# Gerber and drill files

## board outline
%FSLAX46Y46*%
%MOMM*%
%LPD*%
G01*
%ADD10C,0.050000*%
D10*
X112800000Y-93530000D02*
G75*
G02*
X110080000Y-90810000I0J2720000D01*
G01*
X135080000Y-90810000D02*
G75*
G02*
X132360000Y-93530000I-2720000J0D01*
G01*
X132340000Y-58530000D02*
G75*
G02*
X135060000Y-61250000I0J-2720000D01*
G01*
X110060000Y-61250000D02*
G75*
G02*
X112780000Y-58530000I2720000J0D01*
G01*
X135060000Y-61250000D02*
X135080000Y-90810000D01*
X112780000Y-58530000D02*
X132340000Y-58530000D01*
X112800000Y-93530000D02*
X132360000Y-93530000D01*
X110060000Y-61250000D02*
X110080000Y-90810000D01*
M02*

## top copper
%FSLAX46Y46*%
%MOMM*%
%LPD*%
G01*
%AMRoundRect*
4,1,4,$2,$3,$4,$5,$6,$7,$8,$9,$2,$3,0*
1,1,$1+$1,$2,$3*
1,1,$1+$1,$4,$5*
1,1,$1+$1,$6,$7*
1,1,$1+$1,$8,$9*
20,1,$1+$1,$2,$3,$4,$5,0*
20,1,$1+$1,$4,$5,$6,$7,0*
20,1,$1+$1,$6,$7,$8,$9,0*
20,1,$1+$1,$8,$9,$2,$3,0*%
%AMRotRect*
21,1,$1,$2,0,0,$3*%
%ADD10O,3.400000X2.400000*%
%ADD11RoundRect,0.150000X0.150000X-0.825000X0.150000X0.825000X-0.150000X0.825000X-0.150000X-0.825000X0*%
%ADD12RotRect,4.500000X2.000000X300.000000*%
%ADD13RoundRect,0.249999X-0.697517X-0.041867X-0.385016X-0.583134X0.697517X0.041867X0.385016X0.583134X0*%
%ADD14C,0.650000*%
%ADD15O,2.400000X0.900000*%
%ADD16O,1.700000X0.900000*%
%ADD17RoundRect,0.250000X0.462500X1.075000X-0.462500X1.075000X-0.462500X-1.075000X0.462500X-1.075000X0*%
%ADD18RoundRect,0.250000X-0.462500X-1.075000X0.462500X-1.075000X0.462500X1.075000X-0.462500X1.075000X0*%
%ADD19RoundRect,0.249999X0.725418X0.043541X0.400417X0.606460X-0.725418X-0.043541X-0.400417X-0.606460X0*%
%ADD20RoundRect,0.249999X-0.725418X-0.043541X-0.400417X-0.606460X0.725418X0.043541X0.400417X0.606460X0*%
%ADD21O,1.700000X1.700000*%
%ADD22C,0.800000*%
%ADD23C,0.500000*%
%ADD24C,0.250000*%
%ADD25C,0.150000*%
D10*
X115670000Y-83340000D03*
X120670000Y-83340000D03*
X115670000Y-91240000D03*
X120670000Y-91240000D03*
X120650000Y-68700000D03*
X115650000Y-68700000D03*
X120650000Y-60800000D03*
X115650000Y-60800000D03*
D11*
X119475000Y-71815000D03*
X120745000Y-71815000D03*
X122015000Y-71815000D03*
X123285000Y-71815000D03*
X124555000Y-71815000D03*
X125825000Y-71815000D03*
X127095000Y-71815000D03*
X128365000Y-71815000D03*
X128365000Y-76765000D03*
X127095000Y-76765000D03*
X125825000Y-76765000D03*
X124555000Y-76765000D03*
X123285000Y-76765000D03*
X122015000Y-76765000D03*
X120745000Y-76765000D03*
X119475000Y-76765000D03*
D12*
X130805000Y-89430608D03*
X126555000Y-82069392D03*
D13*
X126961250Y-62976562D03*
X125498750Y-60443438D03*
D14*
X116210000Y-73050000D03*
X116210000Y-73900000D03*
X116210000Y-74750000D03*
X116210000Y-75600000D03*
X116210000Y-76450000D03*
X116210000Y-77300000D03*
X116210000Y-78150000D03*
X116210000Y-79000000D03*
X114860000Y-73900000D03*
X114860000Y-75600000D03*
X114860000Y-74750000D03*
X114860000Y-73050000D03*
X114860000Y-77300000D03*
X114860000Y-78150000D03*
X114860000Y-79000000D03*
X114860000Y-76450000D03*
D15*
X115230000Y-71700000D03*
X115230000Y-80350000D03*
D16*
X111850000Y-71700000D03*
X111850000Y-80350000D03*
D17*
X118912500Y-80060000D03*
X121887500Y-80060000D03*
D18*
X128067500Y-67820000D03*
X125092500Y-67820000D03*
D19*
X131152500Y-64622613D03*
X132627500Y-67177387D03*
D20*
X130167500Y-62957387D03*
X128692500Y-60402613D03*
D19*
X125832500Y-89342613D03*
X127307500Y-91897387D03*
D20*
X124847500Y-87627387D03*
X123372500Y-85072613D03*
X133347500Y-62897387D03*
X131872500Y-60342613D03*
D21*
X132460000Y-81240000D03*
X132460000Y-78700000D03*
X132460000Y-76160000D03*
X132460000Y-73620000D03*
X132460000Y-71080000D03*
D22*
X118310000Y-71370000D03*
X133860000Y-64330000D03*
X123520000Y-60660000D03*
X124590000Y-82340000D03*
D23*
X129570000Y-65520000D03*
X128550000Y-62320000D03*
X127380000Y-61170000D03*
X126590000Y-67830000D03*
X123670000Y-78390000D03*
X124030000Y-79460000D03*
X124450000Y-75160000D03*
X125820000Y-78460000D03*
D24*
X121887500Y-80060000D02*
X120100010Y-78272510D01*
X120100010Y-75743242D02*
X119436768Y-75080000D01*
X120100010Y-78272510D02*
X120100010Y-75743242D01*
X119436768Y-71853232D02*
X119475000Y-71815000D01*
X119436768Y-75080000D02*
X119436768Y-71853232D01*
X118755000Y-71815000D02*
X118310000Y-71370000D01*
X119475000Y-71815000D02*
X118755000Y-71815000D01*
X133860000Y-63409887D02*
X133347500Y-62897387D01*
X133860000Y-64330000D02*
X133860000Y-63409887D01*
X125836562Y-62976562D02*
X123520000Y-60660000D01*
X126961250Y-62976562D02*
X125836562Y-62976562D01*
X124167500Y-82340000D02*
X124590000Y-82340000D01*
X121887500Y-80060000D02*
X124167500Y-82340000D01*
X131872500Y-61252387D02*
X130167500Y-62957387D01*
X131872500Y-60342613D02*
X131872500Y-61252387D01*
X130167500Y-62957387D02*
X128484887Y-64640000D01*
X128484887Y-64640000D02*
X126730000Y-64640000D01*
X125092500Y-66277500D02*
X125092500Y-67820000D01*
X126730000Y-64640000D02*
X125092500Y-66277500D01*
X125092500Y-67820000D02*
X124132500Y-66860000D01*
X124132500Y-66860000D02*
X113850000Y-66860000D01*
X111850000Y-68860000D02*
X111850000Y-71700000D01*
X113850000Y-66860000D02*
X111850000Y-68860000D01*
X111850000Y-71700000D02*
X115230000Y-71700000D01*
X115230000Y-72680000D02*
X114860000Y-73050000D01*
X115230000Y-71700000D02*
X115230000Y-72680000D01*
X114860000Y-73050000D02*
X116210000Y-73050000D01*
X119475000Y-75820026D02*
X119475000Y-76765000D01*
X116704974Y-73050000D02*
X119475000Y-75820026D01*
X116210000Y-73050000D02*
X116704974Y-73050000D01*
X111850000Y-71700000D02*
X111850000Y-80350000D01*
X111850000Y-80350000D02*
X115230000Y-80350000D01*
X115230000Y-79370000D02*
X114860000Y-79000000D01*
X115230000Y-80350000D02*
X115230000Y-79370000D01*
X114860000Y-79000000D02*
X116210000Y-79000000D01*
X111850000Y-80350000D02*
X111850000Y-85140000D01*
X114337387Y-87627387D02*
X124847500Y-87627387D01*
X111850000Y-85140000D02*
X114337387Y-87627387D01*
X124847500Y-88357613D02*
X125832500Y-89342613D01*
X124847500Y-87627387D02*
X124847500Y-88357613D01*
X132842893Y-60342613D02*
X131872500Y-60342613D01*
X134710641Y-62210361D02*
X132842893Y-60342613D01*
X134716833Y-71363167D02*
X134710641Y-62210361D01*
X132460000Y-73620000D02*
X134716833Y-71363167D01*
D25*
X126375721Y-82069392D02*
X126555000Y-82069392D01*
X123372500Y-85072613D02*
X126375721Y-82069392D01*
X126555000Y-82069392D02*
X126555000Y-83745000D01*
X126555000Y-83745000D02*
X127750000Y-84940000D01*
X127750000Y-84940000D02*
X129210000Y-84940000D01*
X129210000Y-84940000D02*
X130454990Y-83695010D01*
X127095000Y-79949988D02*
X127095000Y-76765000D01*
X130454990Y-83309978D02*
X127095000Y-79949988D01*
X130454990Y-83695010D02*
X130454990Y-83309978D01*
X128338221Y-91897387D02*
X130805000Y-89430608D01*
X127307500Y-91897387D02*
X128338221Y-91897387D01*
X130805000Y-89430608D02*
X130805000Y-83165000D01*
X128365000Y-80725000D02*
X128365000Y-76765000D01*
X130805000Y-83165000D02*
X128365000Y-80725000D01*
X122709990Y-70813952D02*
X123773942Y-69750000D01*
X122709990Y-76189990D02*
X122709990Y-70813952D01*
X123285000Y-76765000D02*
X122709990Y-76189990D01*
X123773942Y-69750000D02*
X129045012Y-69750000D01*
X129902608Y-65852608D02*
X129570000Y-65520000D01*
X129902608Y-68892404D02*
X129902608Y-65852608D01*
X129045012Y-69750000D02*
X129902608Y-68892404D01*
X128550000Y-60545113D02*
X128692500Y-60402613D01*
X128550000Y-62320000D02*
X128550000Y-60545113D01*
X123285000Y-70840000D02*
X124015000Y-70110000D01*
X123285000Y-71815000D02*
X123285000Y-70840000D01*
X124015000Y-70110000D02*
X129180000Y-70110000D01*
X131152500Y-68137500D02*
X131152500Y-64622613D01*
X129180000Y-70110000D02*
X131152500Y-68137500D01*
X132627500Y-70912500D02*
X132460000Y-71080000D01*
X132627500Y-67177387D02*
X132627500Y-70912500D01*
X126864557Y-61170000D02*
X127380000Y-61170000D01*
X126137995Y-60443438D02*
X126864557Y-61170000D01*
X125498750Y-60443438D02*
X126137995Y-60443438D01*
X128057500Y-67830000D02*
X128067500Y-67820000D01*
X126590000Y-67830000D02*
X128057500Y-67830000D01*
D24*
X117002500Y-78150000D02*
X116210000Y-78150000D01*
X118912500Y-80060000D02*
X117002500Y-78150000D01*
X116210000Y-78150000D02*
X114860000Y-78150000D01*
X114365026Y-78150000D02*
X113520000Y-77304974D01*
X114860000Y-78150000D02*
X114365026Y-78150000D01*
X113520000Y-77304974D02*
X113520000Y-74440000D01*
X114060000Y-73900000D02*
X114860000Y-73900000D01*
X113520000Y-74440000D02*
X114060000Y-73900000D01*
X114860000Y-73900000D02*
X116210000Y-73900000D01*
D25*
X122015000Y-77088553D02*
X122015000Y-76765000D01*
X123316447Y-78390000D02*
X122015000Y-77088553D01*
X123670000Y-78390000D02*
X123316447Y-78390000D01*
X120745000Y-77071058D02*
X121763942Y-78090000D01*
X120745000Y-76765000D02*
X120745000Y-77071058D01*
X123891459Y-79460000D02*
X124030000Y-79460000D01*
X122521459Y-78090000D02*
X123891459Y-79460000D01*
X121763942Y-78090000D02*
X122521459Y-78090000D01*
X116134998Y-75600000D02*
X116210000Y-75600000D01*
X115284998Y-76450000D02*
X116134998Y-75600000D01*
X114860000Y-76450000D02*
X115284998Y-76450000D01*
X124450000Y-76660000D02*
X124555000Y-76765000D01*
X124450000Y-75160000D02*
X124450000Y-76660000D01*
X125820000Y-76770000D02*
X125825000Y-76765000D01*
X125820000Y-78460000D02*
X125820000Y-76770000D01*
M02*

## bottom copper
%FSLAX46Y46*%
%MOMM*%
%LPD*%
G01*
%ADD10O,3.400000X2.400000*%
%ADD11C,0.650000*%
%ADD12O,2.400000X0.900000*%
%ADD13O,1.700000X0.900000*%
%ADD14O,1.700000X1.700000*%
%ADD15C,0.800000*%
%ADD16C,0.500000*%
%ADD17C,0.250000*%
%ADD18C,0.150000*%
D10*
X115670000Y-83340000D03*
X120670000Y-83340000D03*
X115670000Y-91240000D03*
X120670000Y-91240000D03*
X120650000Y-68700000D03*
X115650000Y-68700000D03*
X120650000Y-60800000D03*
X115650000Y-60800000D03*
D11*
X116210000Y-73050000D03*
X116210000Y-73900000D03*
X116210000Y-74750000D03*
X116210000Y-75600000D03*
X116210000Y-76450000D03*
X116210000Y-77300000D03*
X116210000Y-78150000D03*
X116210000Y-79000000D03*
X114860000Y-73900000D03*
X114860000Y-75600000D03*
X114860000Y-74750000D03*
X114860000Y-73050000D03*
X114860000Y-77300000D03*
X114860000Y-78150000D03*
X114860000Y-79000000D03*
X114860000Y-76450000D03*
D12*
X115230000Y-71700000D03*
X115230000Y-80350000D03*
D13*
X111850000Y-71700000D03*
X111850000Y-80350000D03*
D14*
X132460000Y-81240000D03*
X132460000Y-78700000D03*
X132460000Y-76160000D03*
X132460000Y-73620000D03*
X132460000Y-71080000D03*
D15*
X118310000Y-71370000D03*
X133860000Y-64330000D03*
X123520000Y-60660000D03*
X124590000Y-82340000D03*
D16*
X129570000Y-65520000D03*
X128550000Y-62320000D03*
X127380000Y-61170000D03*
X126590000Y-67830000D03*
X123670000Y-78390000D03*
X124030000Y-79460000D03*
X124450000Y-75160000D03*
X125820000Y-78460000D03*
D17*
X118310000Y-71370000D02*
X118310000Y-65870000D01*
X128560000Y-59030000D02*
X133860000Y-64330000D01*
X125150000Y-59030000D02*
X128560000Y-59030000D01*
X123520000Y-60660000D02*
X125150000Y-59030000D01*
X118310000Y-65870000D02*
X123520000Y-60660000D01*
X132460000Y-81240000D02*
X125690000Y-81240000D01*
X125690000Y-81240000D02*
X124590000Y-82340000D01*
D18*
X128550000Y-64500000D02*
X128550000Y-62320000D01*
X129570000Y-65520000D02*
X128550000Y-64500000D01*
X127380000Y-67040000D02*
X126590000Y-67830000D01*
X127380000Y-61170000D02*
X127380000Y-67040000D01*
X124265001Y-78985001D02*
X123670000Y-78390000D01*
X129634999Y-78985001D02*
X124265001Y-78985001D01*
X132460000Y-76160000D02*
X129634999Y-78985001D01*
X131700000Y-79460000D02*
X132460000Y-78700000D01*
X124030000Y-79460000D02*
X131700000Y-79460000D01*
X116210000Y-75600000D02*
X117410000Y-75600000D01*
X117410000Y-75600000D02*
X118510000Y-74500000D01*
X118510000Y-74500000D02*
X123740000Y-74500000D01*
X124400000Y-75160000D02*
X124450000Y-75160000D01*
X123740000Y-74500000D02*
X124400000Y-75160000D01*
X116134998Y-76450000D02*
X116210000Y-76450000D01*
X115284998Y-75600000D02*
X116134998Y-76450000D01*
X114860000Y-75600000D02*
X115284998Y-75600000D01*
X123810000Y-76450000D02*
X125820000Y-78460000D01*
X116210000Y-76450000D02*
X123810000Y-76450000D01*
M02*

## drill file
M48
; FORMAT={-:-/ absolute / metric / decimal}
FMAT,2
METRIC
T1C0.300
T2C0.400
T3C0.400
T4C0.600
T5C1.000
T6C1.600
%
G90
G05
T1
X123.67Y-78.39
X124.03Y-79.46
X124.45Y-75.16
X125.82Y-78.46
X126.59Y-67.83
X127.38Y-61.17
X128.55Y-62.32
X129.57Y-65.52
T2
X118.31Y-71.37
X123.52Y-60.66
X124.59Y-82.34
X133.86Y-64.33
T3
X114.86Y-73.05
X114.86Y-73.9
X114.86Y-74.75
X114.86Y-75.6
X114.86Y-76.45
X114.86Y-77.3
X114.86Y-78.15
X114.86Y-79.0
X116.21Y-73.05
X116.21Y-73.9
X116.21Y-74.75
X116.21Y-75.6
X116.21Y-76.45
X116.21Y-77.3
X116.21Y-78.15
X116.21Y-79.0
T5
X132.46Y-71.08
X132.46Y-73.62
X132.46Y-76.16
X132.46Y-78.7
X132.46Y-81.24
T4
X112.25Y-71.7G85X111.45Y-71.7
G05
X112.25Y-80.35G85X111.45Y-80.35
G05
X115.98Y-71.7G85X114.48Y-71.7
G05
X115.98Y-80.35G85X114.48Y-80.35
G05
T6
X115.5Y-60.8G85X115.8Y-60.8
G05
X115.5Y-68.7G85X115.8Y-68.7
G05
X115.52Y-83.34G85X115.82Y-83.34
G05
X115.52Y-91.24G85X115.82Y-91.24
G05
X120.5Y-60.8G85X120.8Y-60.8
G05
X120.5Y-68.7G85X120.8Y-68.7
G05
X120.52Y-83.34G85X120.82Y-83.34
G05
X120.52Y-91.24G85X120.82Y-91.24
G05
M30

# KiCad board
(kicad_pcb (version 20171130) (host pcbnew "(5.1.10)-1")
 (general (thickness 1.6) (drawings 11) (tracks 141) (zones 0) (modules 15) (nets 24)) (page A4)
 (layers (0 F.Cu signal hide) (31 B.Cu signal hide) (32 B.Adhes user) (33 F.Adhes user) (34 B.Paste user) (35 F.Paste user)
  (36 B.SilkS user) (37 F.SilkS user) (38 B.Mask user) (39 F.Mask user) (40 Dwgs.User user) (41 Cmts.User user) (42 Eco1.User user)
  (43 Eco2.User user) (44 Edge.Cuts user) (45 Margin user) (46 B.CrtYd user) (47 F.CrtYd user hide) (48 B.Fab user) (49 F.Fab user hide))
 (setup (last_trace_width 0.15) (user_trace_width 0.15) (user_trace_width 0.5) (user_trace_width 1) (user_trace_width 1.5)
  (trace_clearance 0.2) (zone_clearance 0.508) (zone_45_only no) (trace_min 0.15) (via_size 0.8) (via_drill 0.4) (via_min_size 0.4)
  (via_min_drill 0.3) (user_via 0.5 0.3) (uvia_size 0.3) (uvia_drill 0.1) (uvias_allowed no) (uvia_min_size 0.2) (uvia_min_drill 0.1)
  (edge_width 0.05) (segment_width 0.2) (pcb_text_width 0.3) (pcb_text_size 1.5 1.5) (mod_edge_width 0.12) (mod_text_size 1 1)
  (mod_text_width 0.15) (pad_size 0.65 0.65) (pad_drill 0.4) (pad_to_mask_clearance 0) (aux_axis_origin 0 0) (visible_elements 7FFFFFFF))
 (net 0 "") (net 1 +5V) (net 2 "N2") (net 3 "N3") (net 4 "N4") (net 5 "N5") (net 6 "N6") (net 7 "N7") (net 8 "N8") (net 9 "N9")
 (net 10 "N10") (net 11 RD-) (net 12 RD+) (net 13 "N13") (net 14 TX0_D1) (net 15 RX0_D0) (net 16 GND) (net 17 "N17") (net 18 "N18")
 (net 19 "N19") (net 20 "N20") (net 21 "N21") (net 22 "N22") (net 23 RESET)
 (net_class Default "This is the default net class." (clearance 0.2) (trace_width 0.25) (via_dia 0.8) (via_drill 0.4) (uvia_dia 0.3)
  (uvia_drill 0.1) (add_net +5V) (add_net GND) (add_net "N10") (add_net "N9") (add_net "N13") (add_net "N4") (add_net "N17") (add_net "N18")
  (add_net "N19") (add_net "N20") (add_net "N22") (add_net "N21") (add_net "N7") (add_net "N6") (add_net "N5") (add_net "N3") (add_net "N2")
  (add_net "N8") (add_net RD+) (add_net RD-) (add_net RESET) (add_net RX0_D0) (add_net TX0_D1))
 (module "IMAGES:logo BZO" (layer B.Cu) (at 123.61 76.22 150)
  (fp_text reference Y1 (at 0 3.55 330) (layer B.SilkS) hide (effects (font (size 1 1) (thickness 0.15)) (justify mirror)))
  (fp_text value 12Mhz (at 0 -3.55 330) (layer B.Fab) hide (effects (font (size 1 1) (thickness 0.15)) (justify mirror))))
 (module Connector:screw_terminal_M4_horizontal (layer F.Cu) (at 115.67 83.54)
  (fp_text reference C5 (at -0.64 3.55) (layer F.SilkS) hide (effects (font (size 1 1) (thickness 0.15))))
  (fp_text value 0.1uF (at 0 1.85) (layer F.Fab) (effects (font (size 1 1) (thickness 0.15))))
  (pad 1 thru_hole oval (at 0 -0.2) (size 3.4 2.4) (drill oval 1.9 1.6) (layers *.Cu *.Mask))
  (pad 2 thru_hole oval (at 5 -0.2) (size 3.4 2.4) (drill oval 1.9 1.6) (layers *.Cu *.Mask))
  (pad 3 thru_hole oval (at 0 7.7) (size 3.4 2.4) (drill oval 1.9 1.6) (layers *.Cu *.Mask))
  (pad 4 thru_hole oval (at 5 7.7) (size 3.4 2.4) (drill oval 1.9 1.6) (layers *.Cu *.Mask)))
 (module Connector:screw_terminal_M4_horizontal (layer F.Cu) (at 115.65 61)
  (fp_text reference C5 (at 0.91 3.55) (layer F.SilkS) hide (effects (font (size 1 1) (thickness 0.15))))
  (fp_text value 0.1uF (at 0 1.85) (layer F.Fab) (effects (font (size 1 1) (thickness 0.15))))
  (pad 4 thru_hole oval (at 5 7.7) (size 3.4 2.4) (drill oval 1.9 1.6) (layers *.Cu *.Mask))
  (pad 3 thru_hole oval (at 0 7.7) (size 3.4 2.4) (drill oval 1.9 1.6) (layers *.Cu *.Mask))
  (pad 2 thru_hole oval (at 5 -0.2) (size 3.4 2.4) (drill oval 1.9 1.6) (layers *.Cu *.Mask))
  (pad 1 thru_hole oval (at 0 -0.2) (size 3.4 2.4) (drill oval 1.9 1.6) (layers *.Cu *.Mask)))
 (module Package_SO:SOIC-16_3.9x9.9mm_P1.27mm (layer F.Cu) (at 123.92 74.29 90)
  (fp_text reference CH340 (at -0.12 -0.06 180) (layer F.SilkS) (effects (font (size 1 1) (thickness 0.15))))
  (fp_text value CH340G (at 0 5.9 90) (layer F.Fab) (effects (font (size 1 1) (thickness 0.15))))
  (pad 16 smd roundrect (at 2.475 -4.445 90) (size 1.95 0.6) (layers F.Cu F.Paste F.Mask) (roundrect_rratio 0.25) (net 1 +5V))
  (pad 15 smd roundrect (at 2.475 -3.175 90) (size 1.95 0.6) (layers F.Cu F.Paste F.Mask) (roundrect_rratio 0.25) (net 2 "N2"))
  (pad 14 smd roundrect (at 2.475 -1.905 90) (size 1.95 0.6) (layers F.Cu F.Paste F.Mask) (roundrect_rratio 0.25) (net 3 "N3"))
  (pad 13 smd roundrect (at 2.475 -0.635 90) (size 1.95 0.6) (layers F.Cu F.Paste F.Mask) (roundrect_rratio 0.25) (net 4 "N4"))
  (pad 12 smd roundrect (at 2.475 0.635 90) (size 1.95 0.6) (layers F.Cu F.Paste F.Mask) (roundrect_rratio 0.25) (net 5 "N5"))
  (pad 11 smd roundrect (at 2.475 1.905 90) (size 1.95 0.6) (layers F.Cu F.Paste F.Mask) (roundrect_rratio 0.25) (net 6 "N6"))
  (pad 10 smd roundrect (at 2.475 3.175 90) (size 1.95 0.6) (layers F.Cu F.Paste F.Mask) (roundrect_rratio 0.25) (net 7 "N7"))
  (pad 9 smd roundrect (at 2.475 4.445 90) (size 1.95 0.6) (layers F.Cu F.Paste F.Mask) (roundrect_rratio 0.25) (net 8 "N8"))
  (pad 8 smd roundrect (at -2.475 4.445 90) (size 1.95 0.6) (layers F.Cu F.Paste F.Mask) (roundrect_rratio 0.25) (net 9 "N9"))
  (pad 7 smd roundrect (at -2.475 3.175 90) (size 1.95 0.6) (layers F.Cu F.Paste F.Mask) (roundrect_rratio 0.25) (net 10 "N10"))
  (pad 6 smd roundrect (at -2.475 1.905 90) (size 1.95 0.6) (layers F.Cu F.Paste F.Mask) (roundrect_rratio 0.25) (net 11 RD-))
  (pad 5 smd roundrect (at -2.475 0.635 90) (size 1.95 0.6) (layers F.Cu F.Paste F.Mask) (roundrect_rratio 0.25) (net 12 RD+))
  (pad 4 smd roundrect (at -2.475 -0.635 90) (size 1.95 0.6) (layers F.Cu F.Paste F.Mask) (roundrect_rratio 0.25) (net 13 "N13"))
  (pad 3 smd roundrect (at -2.475 -1.905 90) (size 1.95 0.6) (layers F.Cu F.Paste F.Mask) (roundrect_rratio 0.25) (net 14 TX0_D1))
  (pad 2 smd roundrect (at -2.475 -3.175 90) (size 1.95 0.6) (layers F.Cu F.Paste F.Mask) (roundrect_rratio 0.25) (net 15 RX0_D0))
  (pad 1 smd roundrect (at -2.475 -4.445 90) (size 1.95 0.6) (layers F.Cu F.Paste F.Mask) (roundrect_rratio 0.25) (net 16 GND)))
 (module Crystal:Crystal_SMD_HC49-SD (layer F.Cu) (at 128.68 85.75 300)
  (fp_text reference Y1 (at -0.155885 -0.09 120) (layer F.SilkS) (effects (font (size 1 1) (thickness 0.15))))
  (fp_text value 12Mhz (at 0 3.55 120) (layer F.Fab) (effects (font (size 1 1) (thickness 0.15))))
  (pad 2 smd rect (at 4.25 0 300) (size 4.5 2) (layers F.Cu F.Paste F.Mask) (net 9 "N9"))
  (pad 1 smd rect (at -4.25 0 300) (size 4.5 2) (layers F.Cu F.Paste F.Mask) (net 10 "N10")))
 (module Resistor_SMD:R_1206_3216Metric (layer F.Cu) (at 126.23 61.71 300)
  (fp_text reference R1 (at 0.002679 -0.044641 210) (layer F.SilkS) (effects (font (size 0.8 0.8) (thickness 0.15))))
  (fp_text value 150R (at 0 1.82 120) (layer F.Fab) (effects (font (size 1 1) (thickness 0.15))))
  (pad 2 smd roundrect (at 1.4625 0 300) (size 1.125 1.75) (layers F.Cu F.Paste F.Mask) (roundrect_rratio 0.2222213333333333) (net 1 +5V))
  (pad 1 smd roundrect (at -1.4625 0 300) (size 1.125 1.75) (layers F.Cu F.Paste F.Mask) (roundrect_rratio 0.2222213333333333)
   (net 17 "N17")))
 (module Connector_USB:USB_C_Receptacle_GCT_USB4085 (layer F.Cu) (at 116.21 73.05 270)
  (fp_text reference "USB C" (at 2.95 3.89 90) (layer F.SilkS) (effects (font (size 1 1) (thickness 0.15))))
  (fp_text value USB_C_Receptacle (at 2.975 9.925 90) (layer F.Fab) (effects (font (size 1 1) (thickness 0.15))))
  (pad A1 thru_hole circle (at 0 0 270) (size 0.65 0.65) (drill 0.4) (layers *.Cu *.Mask) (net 16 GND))
  (pad A4 thru_hole circle (at 0.85 0 270) (size 0.65 0.65) (drill 0.4) (layers *.Cu *.Mask) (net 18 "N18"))
  (pad A5 thru_hole circle (at 1.7 0 270) (size 0.65 0.65) (drill 0.4) (layers *.Cu *.Mask) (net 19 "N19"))
  (pad A6 thru_hole circle (at 2.55 0 270) (size 0.65 0.65) (drill 0.4) (layers *.Cu *.Mask) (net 12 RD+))
  (pad A7 thru_hole circle (at 3.4 0 270) (size 0.65 0.65) (drill 0.4) (layers *.Cu *.Mask) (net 11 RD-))
  (pad A8 thru_hole circle (at 4.25 0 270) (size 0.65 0.65) (drill 0.4) (layers *.Cu *.Mask) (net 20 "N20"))
  (pad A9 thru_hole circle (at 5.1 0 270) (size 0.65 0.65) (drill 0.4) (layers *.Cu *.Mask) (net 18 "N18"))
  (pad A12 thru_hole circle (at 5.95 0 270) (size 0.65 0.65) (drill 0.4) (layers *.Cu *.Mask) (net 16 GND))
  (pad B9 thru_hole circle (at 0.85 1.35 270) (size 0.65 0.65) (drill 0.4) (layers *.Cu *.Mask) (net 18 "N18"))
  (pad B7 thru_hole circle (at 2.55 1.35 270) (size 0.65 0.65) (drill 0.4) (layers *.Cu *.Mask) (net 11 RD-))
  (pad B8 thru_hole circle (at 1.7 1.35 270) (size 0.65 0.65) (drill 0.4) (layers *.Cu *.Mask) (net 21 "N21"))
  (pad B12 thru_hole circle (at 0 1.35 270) (size 0.65 0.65) (drill 0.4) (layers *.Cu *.Mask) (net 16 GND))
  (pad B5 thru_hole circle (at 4.25 1.35 270) (size 0.65 0.65) (drill 0.4) (layers *.Cu *.Mask) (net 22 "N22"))
  (pad B4 thru_hole circle (at 5.1 1.35 270) (size 0.65 0.65) (drill 0.4) (layers *.Cu *.Mask) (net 18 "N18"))
  (pad B1 thru_hole circle (at 5.95 1.35 270) (size 0.65 0.65) (drill 0.4) (layers *.Cu *.Mask) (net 16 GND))
  (pad B6 thru_hole circle (at 3.4 1.35 270) (size 0.65 0.65) (drill 0.4) (layers *.Cu *.Mask) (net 12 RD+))
  (pad S1 thru_hole oval (at -1.35 0.98 270) (size 0.9 2.4) (drill oval 0.6 2.1) (layers *.Cu *.Mask) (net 16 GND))
  (pad S1 thru_hole oval (at 7.3 0.98 270) (size 0.9 2.4) (drill oval 0.6 2.1) (layers *.Cu *.Mask) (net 16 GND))
  (pad S1 thru_hole oval (at -1.35 4.36 270) (size 0.9 1.7) (drill oval 0.6 1.4) (layers *.Cu *.Mask) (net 16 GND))
  (pad S1 thru_hole oval (at 7.3 4.36 270) (size 0.9 1.7) (drill oval 0.6 1.4) (layers *.Cu *.Mask) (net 16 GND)))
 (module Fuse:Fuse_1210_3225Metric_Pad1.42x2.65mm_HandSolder (layer F.Cu) (at 120.4 80.06 180)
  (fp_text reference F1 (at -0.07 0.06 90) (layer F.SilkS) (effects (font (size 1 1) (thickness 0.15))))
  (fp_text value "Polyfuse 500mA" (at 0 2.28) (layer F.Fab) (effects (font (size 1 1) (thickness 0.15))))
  (pad 2 smd roundrect (at 1.4875 0 180) (size 1.425 2.65) (layers F.Cu F.Paste F.Mask) (roundrect_rratio 0.1754385964912281) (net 18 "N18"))
  (pad 1 smd roundrect (at -1.4875 0 180) (size 1.425 2.65) (layers F.Cu F.Paste F.Mask) (roundrect_rratio 0.1754385964912281) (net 1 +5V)))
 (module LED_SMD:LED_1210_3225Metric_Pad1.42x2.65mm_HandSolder (layer F.Cu) (at 126.58 67.82)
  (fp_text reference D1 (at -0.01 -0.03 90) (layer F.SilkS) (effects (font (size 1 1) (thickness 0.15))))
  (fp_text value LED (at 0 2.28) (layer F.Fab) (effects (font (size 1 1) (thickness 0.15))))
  (pad 2 smd roundrect (at 1.4875 0) (size 1.425 2.65) (layers F.Cu F.Paste F.Mask) (roundrect_rratio 0.1754385964912281) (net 17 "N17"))
  (pad 1 smd roundrect (at -1.4875 0) (size 1.425 2.65) (layers F.Cu F.Paste F.Mask) (roundrect_rratio 0.1754385964912281) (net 16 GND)))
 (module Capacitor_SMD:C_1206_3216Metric (layer F.Cu) (at 131.89 65.9 120)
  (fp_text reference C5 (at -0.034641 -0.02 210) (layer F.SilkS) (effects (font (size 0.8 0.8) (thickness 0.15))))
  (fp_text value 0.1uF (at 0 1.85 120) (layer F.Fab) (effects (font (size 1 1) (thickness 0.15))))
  (pad 2 smd roundrect (at 1.475 0 120) (size 1.15 1.8) (layers F.Cu F.Paste F.Mask) (roundrect_rratio 0.2173904347826087) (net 4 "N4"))
  (pad 1 smd roundrect (at -1.475 0 120) (size 1.15 1.8) (layers F.Cu F.Paste F.Mask) (roundrect_rratio 0.2173904347826087) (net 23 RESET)))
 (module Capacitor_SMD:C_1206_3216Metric (layer F.Cu) (at 129.43 61.68 300)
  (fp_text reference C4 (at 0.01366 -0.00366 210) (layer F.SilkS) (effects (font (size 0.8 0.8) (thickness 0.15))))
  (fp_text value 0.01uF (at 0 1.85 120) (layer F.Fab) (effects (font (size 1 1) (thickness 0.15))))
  (pad 2 smd roundrect (at 1.475 0 300) (size 1.15 1.8) (layers F.Cu F.Paste F.Mask) (roundrect_rratio 0.2173904347826087) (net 16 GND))
  (pad 1 smd roundrect (at -1.475 0 300) (size 1.15 1.8) (layers F.Cu F.Paste F.Mask) (roundrect_rratio 0.2173904347826087) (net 13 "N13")))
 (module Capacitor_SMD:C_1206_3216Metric (layer F.Cu) (at 126.57 90.62 120)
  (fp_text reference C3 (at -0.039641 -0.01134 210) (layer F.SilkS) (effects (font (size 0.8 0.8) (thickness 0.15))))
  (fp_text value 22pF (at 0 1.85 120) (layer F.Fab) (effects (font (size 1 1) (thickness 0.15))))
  (pad 2 smd roundrect (at 1.475 0 120) (size 1.15 1.8) (layers F.Cu F.Paste F.Mask) (roundrect_rratio 0.2173904347826087) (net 16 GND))
  (pad 1 smd roundrect (at -1.475 0 120) (size 1.15 1.8) (layers F.Cu F.Paste F.Mask) (roundrect_rratio 0.2173904347826087) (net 9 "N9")))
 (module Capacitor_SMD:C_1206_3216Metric (layer F.Cu) (at 124.11 86.35 300)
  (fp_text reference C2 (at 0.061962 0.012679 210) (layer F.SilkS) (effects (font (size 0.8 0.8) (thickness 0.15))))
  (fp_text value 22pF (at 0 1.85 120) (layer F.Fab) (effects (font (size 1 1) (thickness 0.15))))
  (pad 2 smd roundrect (at 1.475 0 300) (size 1.15 1.8) (layers F.Cu F.Paste F.Mask) (roundrect_rratio 0.2173904347826087) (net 16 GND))
  (pad 1 smd roundrect (at -1.475 0 300) (size 1.15 1.8) (layers F.Cu F.Paste F.Mask) (roundrect_rratio 0.2173904347826087) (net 10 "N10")))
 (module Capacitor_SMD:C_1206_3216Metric (layer F.Cu) (at 132.61 61.62 300)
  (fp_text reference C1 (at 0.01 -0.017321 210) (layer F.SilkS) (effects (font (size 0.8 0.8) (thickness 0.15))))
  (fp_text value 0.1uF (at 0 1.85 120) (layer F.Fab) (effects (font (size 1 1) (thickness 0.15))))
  (pad 2 smd roundrect (at 1.475 0 300) (size 1.15 1.8) (layers F.Cu F.Paste F.Mask) (roundrect_rratio 0.2173904347826087) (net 1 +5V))
  (pad 1 smd roundrect (at -1.475 0 300) (size 1.15 1.8) (layers F.Cu F.Paste F.Mask) (roundrect_rratio 0.2173904347826087) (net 16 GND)))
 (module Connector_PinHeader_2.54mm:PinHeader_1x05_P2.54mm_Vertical (layer F.Cu) (at 132.46 81.24 180)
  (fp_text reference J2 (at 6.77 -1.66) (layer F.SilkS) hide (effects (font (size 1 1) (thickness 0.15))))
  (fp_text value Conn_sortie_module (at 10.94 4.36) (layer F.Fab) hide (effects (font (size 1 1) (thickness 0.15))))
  (pad 1 thru_hole oval (at 0 0 180) (size 1.7 1.7) (drill 1) (layers *.Cu *.Mask) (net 1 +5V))
  (pad 2 thru_hole oval (at 0 2.54 180) (size 1.7 1.7) (drill 1) (layers *.Cu *.Mask) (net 15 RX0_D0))
  (pad 3 thru_hole oval (at 0 5.08 180) (size 1.7 1.7) (drill 1) (layers *.Cu *.Mask) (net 14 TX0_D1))
  (pad 4 thru_hole oval (at 0 7.62 180) (size 1.7 1.7) (drill 1) (layers *.Cu *.Mask) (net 16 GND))
  (pad 5 thru_hole oval (at 0 10.16 180) (size 1.7 1.7) (drill 1) (layers *.Cu *.Mask) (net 23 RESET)))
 (gr_arc (start 112.8 90.81) (end 110.08 90.81) (angle -90) (layer Edge.Cuts) (width 0.05))
 (gr_arc (start 132.36 90.81) (end 132.36 93.53) (angle -90) (layer Edge.Cuts) (width 0.05))
 (gr_arc (start 132.34 61.25) (end 135.06 61.25) (angle -90) (layer Edge.Cuts) (width 0.05))
 (gr_arc (start 112.78 61.25) (end 112.78 58.53) (angle -90) (layer Edge.Cuts) (width 0.05))
 (gr_line (start 135.06 61.25) (end 135.08 90.81) (layer Edge.Cuts) (width 0.05))
 (gr_line (start 112.78 58.53) (end 132.34 58.53) (layer Edge.Cuts) (width 0.05))
 (gr_line (start 112.8 93.53) (end 132.36 93.53) (layer Edge.Cuts) (width 0.05))
 (gr_line (start 110.06 61.25) (end 110.08 90.81) (layer Edge.Cuts) (width 0.05))
 (segment (start 121.8875 80.06) (end 120.10001 78.27251) (width 0.25) (layer F.Cu) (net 1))
 (segment (start 120.10001 75.743242) (end 119.436768 75.08) (width 0.25) (layer F.Cu) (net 1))
 (segment (start 120.10001 78.27251) (end 120.10001 75.743242) (width 0.25) (layer F.Cu) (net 1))
 (segment (start 119.436768 71.853232) (end 119.475 71.815) (width 0.25) (layer F.Cu) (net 1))
 (segment (start 119.436768 75.08) (end 119.436768 71.853232) (width 0.25) (layer F.Cu) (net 1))
 (via (at 118.31 71.37) (size 0.8) (drill 0.4) (layers F.Cu B.Cu) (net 1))
 (segment (start 118.755 71.815) (end 118.31 71.37) (width 0.25) (layer F.Cu) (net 1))
 (segment (start 119.475 71.815) (end 118.755 71.815) (width 0.25) (layer F.Cu) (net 1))
 (segment (start 118.31 71.37) (end 118.31 65.87) (width 0.25) (layer B.Cu) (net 1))
 (via (at 133.86 64.33) (size 0.8) (drill 0.4) (layers F.Cu B.Cu) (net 1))
 (segment (start 128.56 59.03) (end 133.86 64.33) (width 0.25) (layer B.Cu) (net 1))
 (segment (start 125.15 59.03) (end 128.56 59.03) (width 0.25) (layer B.Cu) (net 1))
 (segment (start 133.86 63.409887) (end 133.3475 62.897387) (width 0.25) (layer F.Cu) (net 1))
 (segment (start 133.86 64.33) (end 133.86 63.409887) (width 0.25) (layer F.Cu) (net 1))
 (via (at 123.52 60.66) (size 0.8) (drill 0.4) (layers F.Cu B.Cu) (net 1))
 (segment (start 125.836562 62.976562) (end 123.52 60.66) (width 0.25) (layer F.Cu) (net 1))
 (segment (start 126.96125 62.976562) (end 125.836562 62.976562) (width 0.25) (layer F.Cu) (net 1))
 (segment (start 123.52 60.66) (end 125.15 59.03) (width 0.25) (layer B.Cu) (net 1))
 (segment (start 118.31 65.87) (end 123.52 60.66) (width 0.25) (layer B.Cu) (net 1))
 (via (at 124.59 82.34) (size 0.8) (drill 0.4) (layers F.Cu B.Cu) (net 1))
 (segment (start 124.1675 82.34) (end 124.59 82.34) (width 0.25) (layer F.Cu) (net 1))
 (segment (start 121.8875 80.06) (end 124.1675 82.34) (width 0.25) (layer F.Cu) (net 1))
 (segment (start 132.46 81.24) (end 125.69 81.24) (width 0.25) (layer B.Cu) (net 1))
 (segment (start 125.69 81.24) (end 124.59 82.34) (width 0.25) (layer B.Cu) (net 1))
 (segment (start 131.8725 61.252387) (end 130.1675 62.957387) (width 0.25) (layer F.Cu) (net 16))
 (segment (start 131.8725 60.342613) (end 131.8725 61.252387) (width 0.25) (layer F.Cu) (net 16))
 (segment (start 130.1675 62.957387) (end 128.484887 64.64) (width 0.25) (layer F.Cu) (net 16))
 (segment (start 128.484887 64.64) (end 126.73 64.64) (width 0.25) (layer F.Cu) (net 16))
 (segment (start 125.0925 66.2775) (end 125.0925 67.82) (width 0.25) (layer F.Cu) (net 16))
 (segment (start 126.73 64.64) (end 125.0925 66.2775) (width 0.25) (layer F.Cu) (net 16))
 (segment (start 125.0925 67.82) (end 124.1325 66.86) (width 0.25) (layer F.Cu) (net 16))
 (segment (start 124.1325 66.86) (end 113.85 66.86) (width 0.25) (layer F.Cu) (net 16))
 (segment (start 111.85 68.86) (end 111.85 71.7) (width 0.25) (layer F.Cu) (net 16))
 (segment (start 113.85 66.86) (end 111.85 68.86) (width 0.25) (layer F.Cu) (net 16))
 (segment (start 111.85 71.7) (end 115.23 71.7) (width 0.25) (layer F.Cu) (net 16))
 (segment (start 115.23 72.68) (end 114.86 73.05) (width 0.25) (layer F.Cu) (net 16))
 (segment (start 115.23 71.7) (end 115.23 72.68) (width 0.25) (layer F.Cu) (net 16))
 (segment (start 114.86 73.05) (end 116.21 73.05) (width 0.25) (layer F.Cu) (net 16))
 (segment (start 119.475 75.820026) (end 119.475 76.765) (width 0.25) (layer F.Cu) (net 16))
 (segment (start 116.704974 73.05) (end 119.475 75.820026) (width 0.25) (layer F.Cu) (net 16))
 (segment (start 116.21 73.05) (end 116.704974 73.05) (width 0.25) (layer F.Cu) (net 16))
 (segment (start 111.85 71.7) (end 111.85 80.35) (width 0.25) (layer F.Cu) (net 16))
 (segment (start 111.85 80.35) (end 115.23 80.35) (width 0.25) (layer F.Cu) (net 16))
 (segment (start 115.23 79.37) (end 114.86 79) (width 0.25) (layer F.Cu) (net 16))
 (segment (start 115.23 80.35) (end 115.23 79.37) (width 0.25) (layer F.Cu) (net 16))
 (segment (start 114.86 79) (end 116.21 79) (width 0.25) (layer F.Cu) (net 16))
 (segment (start 111.85 80.35) (end 111.85 85.14) (width 0.25) (layer F.Cu) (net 16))
 (segment (start 114.337387 87.627387) (end 124.8475 87.627387) (width 0.25) (layer F.Cu) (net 16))
 (segment (start 111.85 85.14) (end 114.337387 87.627387) (width 0.25) (layer F.Cu) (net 16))
 (segment (start 124.8475 88.357613) (end 125.8325 89.342613) (width 0.25) (layer F.Cu) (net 16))
 (segment (start 124.8475 87.627387) (end 124.8475 88.357613) (width 0.25) (layer F.Cu) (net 16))
 (segment (start 132.842893 60.342613) (end 131.8725 60.342613) (width 0.25) (layer F.Cu) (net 16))
 (segment (start 134.710641 62.210361) (end 132.842893 60.342613) (width 0.25) (layer F.Cu) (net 16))
 (segment (start 134.716833 71.363167) (end 134.710641 62.210361) (width 0.25) (layer F.Cu) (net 16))
 (segment (start 132.46 73.62) (end 134.716833 71.363167) (width 0.25) (layer F.Cu) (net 16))
 (segment (start 126.375721 82.069392) (end 126.555 82.069392) (width 0.15) (layer F.Cu) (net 10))
 (segment (start 123.3725 85.072613) (end 126.375721 82.069392) (width 0.15) (layer F.Cu) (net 10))
 (segment (start 126.555 82.069392) (end 126.555 83.745) (width 0.15) (layer F.Cu) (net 10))
 (segment (start 126.555 83.745) (end 127.75 84.94) (width 0.15) (layer F.Cu) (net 10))
 (segment (start 127.75 84.94) (end 129.21 84.94) (width 0.15) (layer F.Cu) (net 10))
 (segment (start 129.21 84.94) (end 130.45499 83.69501) (width 0.15) (layer F.Cu) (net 10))
 (segment (start 127.095 79.949988) (end 127.095 76.765) (width 0.15) (layer F.Cu) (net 10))
 (segment (start 130.45499 83.309978) (end 127.095 79.949988) (width 0.15) (layer F.Cu) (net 10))
 (segment (start 130.45499 83.69501) (end 130.45499 83.309978) (width 0.15) (layer F.Cu) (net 10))
 (segment (start 128.338221 91.897387) (end 130.805 89.430608) (width 0.15) (layer F.Cu) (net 9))
 (segment (start 127.3075 91.897387) (end 128.338221 91.897387) (width 0.15) (layer F.Cu) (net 9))
 (segment (start 130.805 89.430608) (end 130.805 83.165) (width 0.15) (layer F.Cu) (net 9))
 (segment (start 128.365 80.725) (end 128.365 76.765) (width 0.15) (layer F.Cu) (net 9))
 (segment (start 130.805 83.165) (end 128.365 80.725) (width 0.15) (layer F.Cu) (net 9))
 (segment (start 122.70999 70.813952) (end 123.773942 69.75) (width 0.15) (layer F.Cu) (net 13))
 (segment (start 122.70999 76.18999) (end 122.70999 70.813952) (width 0.15) (layer F.Cu) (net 13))
 (segment (start 123.285 76.765) (end 122.70999 76.18999) (width 0.15) (layer F.Cu) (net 13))
 (segment (start 123.773942 69.75) (end 129.045012 69.75) (width 0.15) (layer F.Cu) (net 13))
 (via (at 129.57 65.52) (size 0.5) (drill 0.3) (layers F.Cu B.Cu) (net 13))
 (segment (start 129.902608 65.852608) (end 129.57 65.52) (width 0.15) (layer F.Cu) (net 13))
 (segment (start 129.902608 68.892404) (end 129.902608 65.852608) (width 0.15) (layer F.Cu) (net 13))
 (segment (start 129.045012 69.75) (end 129.902608 68.892404) (width 0.15) (layer F.Cu) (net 13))
 (via (at 128.55 62.32) (size 0.5) (drill 0.3) (layers F.Cu B.Cu) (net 13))
 (segment (start 128.55 64.5) (end 128.55 62.32) (width 0.15) (layer B.Cu) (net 13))
 (segment (start 129.57 65.52) (end 128.55 64.5) (width 0.15) (layer B.Cu) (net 13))
 (segment (start 128.55 60.545113) (end 128.6925 60.402613) (width 0.15) (layer F.Cu) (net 13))
 (segment (start 128.55 62.32) (end 128.55 60.545113) (width 0.15) (layer F.Cu) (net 13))
 (segment (start 123.285 70.84) (end 124.015 70.11) (width 0.15) (layer F.Cu) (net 4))
 (segment (start 123.285 71.815) (end 123.285 70.84) (width 0.15) (layer F.Cu) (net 4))
 (segment (start 124.015 70.11) (end 129.18 70.11) (width 0.15) (layer F.Cu) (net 4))
 (segment (start 131.1525 68.1375) (end 131.1525 64.622613) (width 0.15) (layer F.Cu) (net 4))
 (segment (start 129.18 70.11) (end 131.1525 68.1375) (width 0.15) (layer F.Cu) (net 4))
 (segment (start 132.6275 70.9125) (end 132.46 71.08) (width 0.15) (layer F.Cu) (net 23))
 (segment (start 132.6275 67.177387) (end 132.6275 70.9125) (width 0.15) (layer F.Cu) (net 23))
 (via (at 127.38 61.17) (size 0.5) (drill 0.3) (layers F.Cu B.Cu) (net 17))
 (segment (start 126.864557 61.17) (end 127.38 61.17) (width 0.15) (layer F.Cu) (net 17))
 (segment (start 126.137995 60.443438) (end 126.864557 61.17) (width 0.15) (layer F.Cu) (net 17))
 (segment (start 125.49875 60.443438) (end 126.137995 60.443438) (width 0.15) (layer F.Cu) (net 17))
 (via (at 126.59 67.83) (size 0.5) (drill 0.3) (layers F.Cu B.Cu) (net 17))
 (segment (start 127.38 67.04) (end 126.59 67.83) (width 0.15) (layer B.Cu) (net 17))
 (segment (start 127.38 61.17) (end 127.38 67.04) (width 0.15) (layer B.Cu) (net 17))
 (segment (start 128.0575 67.83) (end 128.0675 67.82) (width 0.15) (layer F.Cu) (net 17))
 (segment (start 126.59 67.83) (end 128.0575 67.83) (width 0.15) (layer F.Cu) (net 17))
 (segment (start 117.0025 78.15) (end 116.21 78.15) (width 0.25) (layer F.Cu) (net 18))
 (segment (start 118.9125 80.06) (end 117.0025 78.15) (width 0.25) (layer F.Cu) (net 18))
 (segment (start 116.21 78.15) (end 114.86 78.15) (width 0.25) (layer F.Cu) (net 18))
 (segment (start 114.365026 78.15) (end 113.52 77.304974) (width 0.25) (layer F.Cu) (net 18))
 (segment (start 114.86 78.15) (end 114.365026 78.15) (width 0.25) (layer F.Cu) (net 18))
 (segment (start 113.52 77.304974) (end 113.52 74.44) (width 0.25) (layer F.Cu) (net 18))
 (segment (start 114.06 73.9) (end 114.86 73.9) (width 0.25) (layer F.Cu) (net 18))
 (segment (start 113.52 74.44) (end 114.06 73.9) (width 0.25) (layer F.Cu) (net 18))
 (segment (start 114.86 73.9) (end 116.21 73.9) (width 0.25) (layer F.Cu) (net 18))
 (via (at 123.67 78.39) (size 0.5) (drill 0.3) (layers F.Cu B.Cu) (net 14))
 (segment (start 124.265001 78.985001) (end 123.67 78.39) (width 0.15) (layer B.Cu) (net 14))
 (segment (start 129.634999 78.985001) (end 124.265001 78.985001) (width 0.15) (layer B.Cu) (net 14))
 (segment (start 132.46 76.16) (end 129.634999 78.985001) (width 0.15) (layer B.Cu) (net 14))
 (segment (start 122.015 77.088553) (end 122.015 76.765) (width 0.15) (layer F.Cu) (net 14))
 (segment (start 123.316447 78.39) (end 122.015 77.088553) (width 0.15) (layer F.Cu) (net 14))
 (segment (start 123.67 78.39) (end 123.316447 78.39) (width 0.15) (layer F.Cu) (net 14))
 (segment (start 120.745 77.071058) (end 121.763942 78.09) (width 0.15) (layer F.Cu) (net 15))
 (segment (start 120.745 76.765) (end 120.745 77.071058) (width 0.15) (layer F.Cu) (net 15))
 (segment (start 123.891459 79.46) (end 124.03 79.46) (width 0.15) (layer F.Cu) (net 15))
 (via (at 124.03 79.46) (size 0.5) (drill 0.3) (layers F.Cu B.Cu) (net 15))
 (segment (start 122.521459 78.09) (end 123.891459 79.46) (width 0.15) (layer F.Cu) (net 15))
 (segment (start 121.763942 78.09) (end 122.521459 78.09) (width 0.15) (layer F.Cu) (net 15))
 (segment (start 131.7 79.46) (end 132.46 78.7) (width 0.15) (layer B.Cu) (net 15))
 (segment (start 124.03 79.46) (end 131.7 79.46) (width 0.15) (layer B.Cu) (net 15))
 (segment (start 116.134998 75.6) (end 116.21 75.6) (width 0.15) (layer F.Cu) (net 12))
 (segment (start 115.284998 76.45) (end 116.134998 75.6) (width 0.15) (layer F.Cu) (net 12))
 (segment (start 114.86 76.45) (end 115.284998 76.45) (width 0.15) (layer F.Cu) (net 12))
 (segment (start 116.21 75.6) (end 117.41 75.6) (width 0.15) (layer B.Cu) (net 12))
 (segment (start 117.41 75.6) (end 118.51 74.5) (width 0.15) (layer B.Cu) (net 12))
 (segment (start 118.51 74.5) (end 123.74 74.5) (width 0.15) (layer B.Cu) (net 12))
 (via (at 124.45 75.16) (size 0.5) (drill 0.3) (layers F.Cu B.Cu) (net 12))
 (segment (start 124.4 75.16) (end 124.45 75.16) (width 0.15) (layer B.Cu) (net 12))
 (segment (start 123.74 74.5) (end 124.4 75.16) (width 0.15) (layer B.Cu) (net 12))
 (segment (start 124.45 76.66) (end 124.555 76.765) (width 0.15) (layer F.Cu) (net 12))
 (segment (start 124.45 75.16) (end 124.45 76.66) (width 0.15) (layer F.Cu) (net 12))
 (segment (start 116.134998 76.45) (end 116.21 76.45) (width 0.15) (layer B.Cu) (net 11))
 (segment (start 115.284998 75.6) (end 116.134998 76.45) (width 0.15) (layer B.Cu) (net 11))
 (segment (start 114.86 75.6) (end 115.284998 75.6) (width 0.15) (layer B.Cu) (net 11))
 (via (at 125.82 78.46) (size 0.5) (drill 0.3) (layers F.Cu B.Cu) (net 11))
 (segment (start 123.81 76.45) (end 125.82 78.46) (width 0.15) (layer B.Cu) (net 11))
 (segment (start 116.21 76.45) (end 123.81 76.45) (width 0.15) (layer B.Cu) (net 11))
 (segment (start 125.82 76.77) (end 125.825 76.765) (width 0.15) (layer F.Cu) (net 11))
 (segment (start 125.82 78.46) (end 125.82 76.77) (width 0.15) (layer F.Cu) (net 11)))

